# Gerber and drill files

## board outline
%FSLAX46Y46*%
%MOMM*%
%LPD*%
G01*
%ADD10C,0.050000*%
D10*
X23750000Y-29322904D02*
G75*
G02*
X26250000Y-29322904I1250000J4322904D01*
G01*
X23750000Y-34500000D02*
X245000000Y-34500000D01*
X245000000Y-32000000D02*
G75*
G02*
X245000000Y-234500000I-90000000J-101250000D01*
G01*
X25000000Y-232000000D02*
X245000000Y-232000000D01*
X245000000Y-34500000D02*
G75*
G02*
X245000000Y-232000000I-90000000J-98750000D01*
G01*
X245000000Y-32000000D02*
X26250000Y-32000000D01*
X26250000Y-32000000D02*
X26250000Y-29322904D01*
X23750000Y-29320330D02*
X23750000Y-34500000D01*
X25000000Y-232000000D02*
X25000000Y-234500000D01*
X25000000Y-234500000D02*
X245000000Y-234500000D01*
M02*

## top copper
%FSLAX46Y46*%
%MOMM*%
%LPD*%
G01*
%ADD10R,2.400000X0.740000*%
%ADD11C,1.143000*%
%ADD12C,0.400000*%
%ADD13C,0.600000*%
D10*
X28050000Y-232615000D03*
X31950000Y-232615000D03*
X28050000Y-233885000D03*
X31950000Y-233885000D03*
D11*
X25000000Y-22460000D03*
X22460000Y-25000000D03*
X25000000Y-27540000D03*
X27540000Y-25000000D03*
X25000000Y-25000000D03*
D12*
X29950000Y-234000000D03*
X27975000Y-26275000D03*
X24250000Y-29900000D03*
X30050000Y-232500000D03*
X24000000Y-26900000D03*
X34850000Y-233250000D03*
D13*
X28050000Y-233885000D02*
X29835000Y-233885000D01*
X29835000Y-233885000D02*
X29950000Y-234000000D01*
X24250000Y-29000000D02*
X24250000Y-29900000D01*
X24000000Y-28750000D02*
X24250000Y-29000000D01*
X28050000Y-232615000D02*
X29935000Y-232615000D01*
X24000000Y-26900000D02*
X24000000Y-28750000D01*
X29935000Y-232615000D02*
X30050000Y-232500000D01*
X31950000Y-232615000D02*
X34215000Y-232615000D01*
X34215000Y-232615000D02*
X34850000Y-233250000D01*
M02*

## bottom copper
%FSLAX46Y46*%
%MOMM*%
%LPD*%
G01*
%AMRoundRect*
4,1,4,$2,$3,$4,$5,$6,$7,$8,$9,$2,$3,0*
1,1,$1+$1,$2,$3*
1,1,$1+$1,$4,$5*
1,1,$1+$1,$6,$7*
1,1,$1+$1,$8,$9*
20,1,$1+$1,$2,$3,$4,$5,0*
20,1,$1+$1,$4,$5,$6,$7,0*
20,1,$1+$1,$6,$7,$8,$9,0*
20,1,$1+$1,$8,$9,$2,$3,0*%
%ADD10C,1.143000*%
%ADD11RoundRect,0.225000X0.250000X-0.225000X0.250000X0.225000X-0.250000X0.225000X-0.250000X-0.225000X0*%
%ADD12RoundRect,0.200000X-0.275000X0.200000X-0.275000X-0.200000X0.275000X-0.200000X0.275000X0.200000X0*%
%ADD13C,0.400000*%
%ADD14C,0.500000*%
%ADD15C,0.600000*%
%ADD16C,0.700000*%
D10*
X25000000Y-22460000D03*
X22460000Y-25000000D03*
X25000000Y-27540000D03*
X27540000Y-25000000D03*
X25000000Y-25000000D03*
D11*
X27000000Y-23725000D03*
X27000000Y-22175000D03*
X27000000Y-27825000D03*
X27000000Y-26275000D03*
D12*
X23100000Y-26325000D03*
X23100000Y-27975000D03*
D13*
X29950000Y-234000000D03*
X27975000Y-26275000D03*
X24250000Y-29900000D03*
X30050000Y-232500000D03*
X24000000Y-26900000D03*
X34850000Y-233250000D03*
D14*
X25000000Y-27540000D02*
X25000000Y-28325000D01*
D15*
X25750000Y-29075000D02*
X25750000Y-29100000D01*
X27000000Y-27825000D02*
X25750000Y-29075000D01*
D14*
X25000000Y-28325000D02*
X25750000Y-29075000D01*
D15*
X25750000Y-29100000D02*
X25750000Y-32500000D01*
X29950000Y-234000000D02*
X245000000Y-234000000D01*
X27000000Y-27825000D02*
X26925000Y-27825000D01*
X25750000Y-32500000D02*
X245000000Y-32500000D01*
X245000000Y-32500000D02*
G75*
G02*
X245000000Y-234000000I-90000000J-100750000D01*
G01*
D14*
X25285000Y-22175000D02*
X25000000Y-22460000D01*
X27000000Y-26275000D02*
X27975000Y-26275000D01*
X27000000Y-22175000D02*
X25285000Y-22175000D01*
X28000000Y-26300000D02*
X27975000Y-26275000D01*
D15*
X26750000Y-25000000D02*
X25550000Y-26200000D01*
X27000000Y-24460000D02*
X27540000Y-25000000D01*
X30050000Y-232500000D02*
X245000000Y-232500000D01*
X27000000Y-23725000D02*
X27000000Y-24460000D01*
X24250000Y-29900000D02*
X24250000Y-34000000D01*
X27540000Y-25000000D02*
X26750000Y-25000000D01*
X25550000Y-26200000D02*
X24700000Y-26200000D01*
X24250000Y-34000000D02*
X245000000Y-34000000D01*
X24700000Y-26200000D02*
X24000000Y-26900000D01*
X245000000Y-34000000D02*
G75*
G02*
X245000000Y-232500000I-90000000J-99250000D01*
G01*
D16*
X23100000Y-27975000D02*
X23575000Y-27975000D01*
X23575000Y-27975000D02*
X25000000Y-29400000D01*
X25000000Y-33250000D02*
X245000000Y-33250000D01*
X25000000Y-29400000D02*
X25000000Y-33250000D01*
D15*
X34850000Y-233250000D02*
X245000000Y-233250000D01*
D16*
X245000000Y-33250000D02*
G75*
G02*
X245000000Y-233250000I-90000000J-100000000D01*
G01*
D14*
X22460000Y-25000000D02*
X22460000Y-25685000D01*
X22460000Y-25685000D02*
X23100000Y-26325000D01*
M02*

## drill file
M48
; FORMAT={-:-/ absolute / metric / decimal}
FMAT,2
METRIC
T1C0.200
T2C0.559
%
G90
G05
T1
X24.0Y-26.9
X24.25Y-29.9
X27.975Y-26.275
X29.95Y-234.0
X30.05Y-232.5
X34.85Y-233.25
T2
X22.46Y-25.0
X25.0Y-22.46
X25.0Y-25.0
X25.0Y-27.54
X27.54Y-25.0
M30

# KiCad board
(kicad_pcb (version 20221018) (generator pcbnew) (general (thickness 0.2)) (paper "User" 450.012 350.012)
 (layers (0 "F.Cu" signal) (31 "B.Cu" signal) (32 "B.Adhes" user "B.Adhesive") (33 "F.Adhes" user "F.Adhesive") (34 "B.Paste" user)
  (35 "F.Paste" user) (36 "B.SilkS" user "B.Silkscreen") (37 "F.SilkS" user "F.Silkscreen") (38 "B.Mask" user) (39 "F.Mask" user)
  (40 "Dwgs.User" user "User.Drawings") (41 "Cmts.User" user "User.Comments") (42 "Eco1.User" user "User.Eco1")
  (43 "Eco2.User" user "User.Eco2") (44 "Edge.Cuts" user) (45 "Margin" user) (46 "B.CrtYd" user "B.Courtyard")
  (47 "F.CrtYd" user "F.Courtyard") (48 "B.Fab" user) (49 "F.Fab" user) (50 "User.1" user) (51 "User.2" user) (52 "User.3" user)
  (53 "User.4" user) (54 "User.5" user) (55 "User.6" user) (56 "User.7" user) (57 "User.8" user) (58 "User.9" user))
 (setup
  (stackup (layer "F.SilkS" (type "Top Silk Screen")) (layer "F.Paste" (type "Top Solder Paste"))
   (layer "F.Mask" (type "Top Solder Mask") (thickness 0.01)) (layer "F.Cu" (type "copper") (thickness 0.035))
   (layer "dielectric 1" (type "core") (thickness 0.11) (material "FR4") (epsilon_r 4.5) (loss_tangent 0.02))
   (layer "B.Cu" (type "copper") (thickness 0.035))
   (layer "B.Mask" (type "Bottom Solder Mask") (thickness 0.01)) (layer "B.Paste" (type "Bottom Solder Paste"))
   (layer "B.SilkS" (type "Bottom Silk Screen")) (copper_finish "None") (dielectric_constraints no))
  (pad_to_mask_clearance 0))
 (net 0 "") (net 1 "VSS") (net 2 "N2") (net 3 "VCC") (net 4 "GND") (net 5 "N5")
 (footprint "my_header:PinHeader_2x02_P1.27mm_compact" (layer "F.Cu") (at 30 233.25)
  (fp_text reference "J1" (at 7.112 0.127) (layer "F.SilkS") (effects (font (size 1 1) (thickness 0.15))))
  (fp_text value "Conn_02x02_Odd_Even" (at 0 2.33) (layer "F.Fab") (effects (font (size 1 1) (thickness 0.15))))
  (pad "1" smd rect (at -1.95 -0.635) (size 2.4 0.74) (layers "F.Cu" "F.Paste" "F.Mask") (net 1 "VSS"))
  (pad "2" smd rect (at 1.95 -0.635) (size 2.4 0.74) (layers "F.Cu" "F.Paste" "F.Mask") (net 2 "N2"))
  (pad "3" smd rect (at -1.95 0.635) (size 2.4 0.74) (layers "F.Cu" "F.Paste" "F.Mask") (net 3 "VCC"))
  (pad "4" smd rect (at 1.95 0.635) (size 2.4 0.74) (layers "F.Cu" "F.Paste" "F.Mask") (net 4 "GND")))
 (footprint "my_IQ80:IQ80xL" (layer "F.Cu") (at 25 25 90)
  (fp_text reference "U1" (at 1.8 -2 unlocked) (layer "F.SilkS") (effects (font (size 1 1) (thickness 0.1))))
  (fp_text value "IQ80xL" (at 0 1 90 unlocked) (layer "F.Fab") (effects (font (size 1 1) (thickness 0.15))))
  (pad "1" thru_hole circle (at 2.54 0 90) (size 1.143 1.143) (drill 0.5588) (layers "*.Cu" "*.Mask") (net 4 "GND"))
  (pad "2" thru_hole circle (at 0 -2.54 90) (size 1.143 1.143) (drill 0.5588) (layers "*.Cu" "*.Mask") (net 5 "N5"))
  (pad "3" thru_hole circle (at -2.54 0 90) (size 1.143 1.143) (drill 0.5588) (layers "*.Cu" "*.Mask") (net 3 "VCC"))
  (pad "4" thru_hole circle (at 0 2.54 90) (size 1.143 1.143) (drill 0.5588) (layers "*.Cu" "*.Mask") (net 1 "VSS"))
  (pad "5" thru_hole circle (at 0 0 90) (size 1.143 1.143) (drill 0.5588) (layers "*.Cu" "*.Mask") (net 4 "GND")))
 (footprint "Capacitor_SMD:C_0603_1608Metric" (layer "B.Cu") (at 27 22.95 90)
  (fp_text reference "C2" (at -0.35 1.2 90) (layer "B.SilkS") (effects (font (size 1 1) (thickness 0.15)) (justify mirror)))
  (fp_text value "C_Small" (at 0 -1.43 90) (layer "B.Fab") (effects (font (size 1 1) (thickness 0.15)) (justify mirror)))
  (pad "1" smd roundrect (at -0.775 0 90) (size 0.9 0.95) (layers "B.Cu" "B.Paste" "B.Mask") (roundrect_rratio 0.25) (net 1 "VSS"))
  (pad "2" smd roundrect (at 0.775 0 90) (size 0.9 0.95) (layers "B.Cu" "B.Paste" "B.Mask") (roundrect_rratio 0.25) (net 4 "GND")))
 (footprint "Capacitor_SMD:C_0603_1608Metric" (layer "B.Cu") (at 27 27.05 90)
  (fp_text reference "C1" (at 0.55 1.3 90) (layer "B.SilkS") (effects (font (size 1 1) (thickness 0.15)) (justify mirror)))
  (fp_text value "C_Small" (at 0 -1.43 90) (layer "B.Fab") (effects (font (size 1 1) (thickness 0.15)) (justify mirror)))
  (pad "1" smd roundrect (at -0.775 0 90) (size 0.9 0.95) (layers "B.Cu" "B.Paste" "B.Mask") (roundrect_rratio 0.25) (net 3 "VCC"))
  (pad "2" smd roundrect (at 0.775 0 90) (size 0.9 0.95) (layers "B.Cu" "B.Paste" "B.Mask") (roundrect_rratio 0.25) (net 4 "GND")))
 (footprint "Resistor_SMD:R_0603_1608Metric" (layer "B.Cu") (at 23.1 27.15 -90)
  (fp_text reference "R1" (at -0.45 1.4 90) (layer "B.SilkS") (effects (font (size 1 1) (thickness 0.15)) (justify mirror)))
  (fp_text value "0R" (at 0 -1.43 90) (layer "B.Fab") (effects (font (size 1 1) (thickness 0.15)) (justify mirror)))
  (pad "1" smd roundrect (at -0.825 0 270) (size 0.8 0.95) (layers "B.Cu" "B.Paste" "B.Mask") (roundrect_rratio 0.25) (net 5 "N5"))
  (pad "2" smd roundrect (at 0.825 0 270) (size 0.8 0.95) (layers "B.Cu" "B.Paste" "B.Mask") (roundrect_rratio 0.25) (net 2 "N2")))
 (gr_arc (start 23.75 29.322904) (mid 25 20.5) (end 26.25 29.322904) (stroke (width 0.05) (type solid)) (layer "Edge.Cuts"))
 (gr_line (start 23.75 34.5) (end 245 34.5) (stroke (width 0.05) (type solid)) (layer "Edge.Cuts"))
 (gr_arc (start 245 32) (mid 256.25 43.25) (end 245 234.5) (stroke (width 0.05) (type solid)) (layer "Edge.Cuts"))
 (gr_line (start 25 232) (end 245 232) (stroke (width 0.05) (type solid)) (layer "Edge.Cuts"))
 (gr_arc (start 245 34.5) (mid 253.75 43.25) (end 245 232) (stroke (width 0.05) (type solid)) (layer "Edge.Cuts"))
 (gr_line (start 245 32) (end 26.25 32) (stroke (width 0.05) (type solid)) (layer "Edge.Cuts"))
 (gr_line (start 26.25 32) (end 26.25 29.322904) (stroke (width 0.05) (type solid)) (layer "Edge.Cuts"))
 (gr_line (start 23.75 29.32033) (end 23.75 34.5) (stroke (width 0.05) (type solid)) (layer "Edge.Cuts"))
 (gr_line (start 25 232) (end 25 234.5) (stroke (width 0.05) (type solid)) (layer "Edge.Cuts"))
 (gr_line (start 25 234.5) (end 245 234.5) (stroke (width 0.05) (type solid)) (layer "Edge.Cuts"))
 (segment (start 28.05 233.885) (end 29.835 233.885) (width 0.6) (layer "F.Cu") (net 3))
 (segment (start 29.835 233.885) (end 29.95 234) (width 0.6) (layer "F.Cu") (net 3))
 (via (at 29.95 234) (size 0.4) (drill 0.2) (layers "F.Cu" "B.Cu") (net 3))
 (segment (start 25 27.54) (end 25 28.325) (width 0.5) (layer "B.Cu") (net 3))
 (segment (start 25.75 29.075) (end 25.75 29.1) (width 0.6) (layer "B.Cu") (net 3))
 (segment (start 27 27.825) (end 25.75 29.075) (width 0.6) (layer "B.Cu") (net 3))
 (segment (start 25 28.325) (end 25.75 29.075) (width 0.5) (layer "B.Cu") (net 3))
 (segment (start 25.75 29.1) (end 25.75 32.5) (width 0.6) (layer "B.Cu") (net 3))
 (segment (start 29.95 234) (end 245 234) (width 0.6) (layer "B.Cu") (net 3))
 (segment (start 27 27.825) (end 26.925 27.825) (width 0.6) (layer "B.Cu") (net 3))
 (segment (start 25.75 32.5) (end 245 32.5) (width 0.6) (layer "B.Cu") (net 3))
 (arc (start 245 32.5) (mid 255.75 43.25) (end 245 234) (width 0.6) (layer "B.Cu") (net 3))
 (via (at 27.975 26.275) (size 0.4) (drill 0.2) (layers "F.Cu" "B.Cu") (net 4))
 (segment (start 25.285 22.175) (end 25 22.46) (width 0.5) (layer "B.Cu") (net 4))
 (segment (start 27 26.275) (end 27.975 26.275) (width 0.5) (layer "B.Cu") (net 4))
 (segment (start 27 22.175) (end 25.285 22.175) (width 0.5) (layer "B.Cu") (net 4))
 (segment (start 28 26.3) (end 27.975 26.275) (width 0.5) (layer "B.Cu") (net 4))
 (segment (start 24.25 29) (end 24.25 29.9) (width 0.6) (layer "F.Cu") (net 1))
 (segment (start 24 28.75) (end 24.25 29) (width 0.6) (layer "F.Cu") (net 1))
 (segment (start 28.05 232.615) (end 29.935 232.615) (width 0.6) (layer "F.Cu") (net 1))
 (segment (start 24 26.9) (end 24 28.75) (width 0.6) (layer "F.Cu") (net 1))
 (segment (start 29.935 232.615) (end 30.05 232.5) (width 0.6) (layer "F.Cu") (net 1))
 (via (at 24.25 29.9) (size 0.4) (drill 0.2) (layers "F.Cu" "B.Cu") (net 1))
 (via (at 30.05 232.5) (size 0.4) (drill 0.2) (layers "F.Cu" "B.Cu") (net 1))
 (via (at 24 26.9) (size 0.4) (drill 0.2) (layers "F.Cu" "B.Cu") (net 1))
 (segment (start 26.75 25) (end 25.55 26.2) (width 0.6) (layer "B.Cu") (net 1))
 (segment (start 27 24.46) (end 27.54 25) (width 0.6) (layer "B.Cu") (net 1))
 (segment (start 30.05 232.5) (end 245 232.5) (width 0.6) (layer "B.Cu") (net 1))
 (segment (start 27 23.725) (end 27 24.46) (width 0.6) (layer "B.Cu") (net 1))
 (segment (start 24.25 29.9) (end 24.25 34) (width 0.6) (layer "B.Cu") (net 1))
 (segment (start 27.54 25) (end 26.75 25) (width 0.6) (layer "B.Cu") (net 1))
 (segment (start 25.55 26.2) (end 24.7 26.2) (width 0.6) (layer "B.Cu") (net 1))
 (segment (start 24.25 34) (end 245 34) (width 0.6) (layer "B.Cu") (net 1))
 (segment (start 24.7 26.2) (end 24 26.9) (width 0.6) (layer "B.Cu") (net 1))
 (arc (start 245 34) (mid 254.25 43.25) (end 245 232.5) (width 0.6) (layer "B.Cu") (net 1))
 (segment (start 31.95 232.615) (end 34.215 232.615) (width 0.6) (layer "F.Cu") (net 2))
 (segment (start 34.215 232.615) (end 34.85 233.25) (width 0.6) (layer "F.Cu") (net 2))
 (via (at 34.85 233.25) (size 0.4) (drill 0.2) (layers "F.Cu" "B.Cu") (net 2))
 (segment (start 23.1 27.975) (end 23.575 27.975) (width 0.7) (layer "B.Cu") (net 2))
 (segment (start 23.575 27.975) (end 25 29.4) (width 0.7) (layer "B.Cu") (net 2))
 (segment (start 25 33.25) (end 245 33.25) (width 0.7) (layer "B.Cu") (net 2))
 (segment (start 25 29.4) (end 25 33.25) (width 0.7) (layer "B.Cu") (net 2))
 (segment (start 34.85 233.25) (end 245 233.25) (width 0.6) (layer "B.Cu") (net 2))
 (arc (start 245 33.25) (mid 255. 43.25) (end 245 233.25) (width 0.7) (layer "B.Cu") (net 2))
 (segment (start 22.46 25) (end 22.46 25.685) (width 0.5) (layer "B.Cu") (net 5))
 (segment (start 22.46 25.685) (end 23.1 26.325) (width 0.5) (layer "B.Cu") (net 5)))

